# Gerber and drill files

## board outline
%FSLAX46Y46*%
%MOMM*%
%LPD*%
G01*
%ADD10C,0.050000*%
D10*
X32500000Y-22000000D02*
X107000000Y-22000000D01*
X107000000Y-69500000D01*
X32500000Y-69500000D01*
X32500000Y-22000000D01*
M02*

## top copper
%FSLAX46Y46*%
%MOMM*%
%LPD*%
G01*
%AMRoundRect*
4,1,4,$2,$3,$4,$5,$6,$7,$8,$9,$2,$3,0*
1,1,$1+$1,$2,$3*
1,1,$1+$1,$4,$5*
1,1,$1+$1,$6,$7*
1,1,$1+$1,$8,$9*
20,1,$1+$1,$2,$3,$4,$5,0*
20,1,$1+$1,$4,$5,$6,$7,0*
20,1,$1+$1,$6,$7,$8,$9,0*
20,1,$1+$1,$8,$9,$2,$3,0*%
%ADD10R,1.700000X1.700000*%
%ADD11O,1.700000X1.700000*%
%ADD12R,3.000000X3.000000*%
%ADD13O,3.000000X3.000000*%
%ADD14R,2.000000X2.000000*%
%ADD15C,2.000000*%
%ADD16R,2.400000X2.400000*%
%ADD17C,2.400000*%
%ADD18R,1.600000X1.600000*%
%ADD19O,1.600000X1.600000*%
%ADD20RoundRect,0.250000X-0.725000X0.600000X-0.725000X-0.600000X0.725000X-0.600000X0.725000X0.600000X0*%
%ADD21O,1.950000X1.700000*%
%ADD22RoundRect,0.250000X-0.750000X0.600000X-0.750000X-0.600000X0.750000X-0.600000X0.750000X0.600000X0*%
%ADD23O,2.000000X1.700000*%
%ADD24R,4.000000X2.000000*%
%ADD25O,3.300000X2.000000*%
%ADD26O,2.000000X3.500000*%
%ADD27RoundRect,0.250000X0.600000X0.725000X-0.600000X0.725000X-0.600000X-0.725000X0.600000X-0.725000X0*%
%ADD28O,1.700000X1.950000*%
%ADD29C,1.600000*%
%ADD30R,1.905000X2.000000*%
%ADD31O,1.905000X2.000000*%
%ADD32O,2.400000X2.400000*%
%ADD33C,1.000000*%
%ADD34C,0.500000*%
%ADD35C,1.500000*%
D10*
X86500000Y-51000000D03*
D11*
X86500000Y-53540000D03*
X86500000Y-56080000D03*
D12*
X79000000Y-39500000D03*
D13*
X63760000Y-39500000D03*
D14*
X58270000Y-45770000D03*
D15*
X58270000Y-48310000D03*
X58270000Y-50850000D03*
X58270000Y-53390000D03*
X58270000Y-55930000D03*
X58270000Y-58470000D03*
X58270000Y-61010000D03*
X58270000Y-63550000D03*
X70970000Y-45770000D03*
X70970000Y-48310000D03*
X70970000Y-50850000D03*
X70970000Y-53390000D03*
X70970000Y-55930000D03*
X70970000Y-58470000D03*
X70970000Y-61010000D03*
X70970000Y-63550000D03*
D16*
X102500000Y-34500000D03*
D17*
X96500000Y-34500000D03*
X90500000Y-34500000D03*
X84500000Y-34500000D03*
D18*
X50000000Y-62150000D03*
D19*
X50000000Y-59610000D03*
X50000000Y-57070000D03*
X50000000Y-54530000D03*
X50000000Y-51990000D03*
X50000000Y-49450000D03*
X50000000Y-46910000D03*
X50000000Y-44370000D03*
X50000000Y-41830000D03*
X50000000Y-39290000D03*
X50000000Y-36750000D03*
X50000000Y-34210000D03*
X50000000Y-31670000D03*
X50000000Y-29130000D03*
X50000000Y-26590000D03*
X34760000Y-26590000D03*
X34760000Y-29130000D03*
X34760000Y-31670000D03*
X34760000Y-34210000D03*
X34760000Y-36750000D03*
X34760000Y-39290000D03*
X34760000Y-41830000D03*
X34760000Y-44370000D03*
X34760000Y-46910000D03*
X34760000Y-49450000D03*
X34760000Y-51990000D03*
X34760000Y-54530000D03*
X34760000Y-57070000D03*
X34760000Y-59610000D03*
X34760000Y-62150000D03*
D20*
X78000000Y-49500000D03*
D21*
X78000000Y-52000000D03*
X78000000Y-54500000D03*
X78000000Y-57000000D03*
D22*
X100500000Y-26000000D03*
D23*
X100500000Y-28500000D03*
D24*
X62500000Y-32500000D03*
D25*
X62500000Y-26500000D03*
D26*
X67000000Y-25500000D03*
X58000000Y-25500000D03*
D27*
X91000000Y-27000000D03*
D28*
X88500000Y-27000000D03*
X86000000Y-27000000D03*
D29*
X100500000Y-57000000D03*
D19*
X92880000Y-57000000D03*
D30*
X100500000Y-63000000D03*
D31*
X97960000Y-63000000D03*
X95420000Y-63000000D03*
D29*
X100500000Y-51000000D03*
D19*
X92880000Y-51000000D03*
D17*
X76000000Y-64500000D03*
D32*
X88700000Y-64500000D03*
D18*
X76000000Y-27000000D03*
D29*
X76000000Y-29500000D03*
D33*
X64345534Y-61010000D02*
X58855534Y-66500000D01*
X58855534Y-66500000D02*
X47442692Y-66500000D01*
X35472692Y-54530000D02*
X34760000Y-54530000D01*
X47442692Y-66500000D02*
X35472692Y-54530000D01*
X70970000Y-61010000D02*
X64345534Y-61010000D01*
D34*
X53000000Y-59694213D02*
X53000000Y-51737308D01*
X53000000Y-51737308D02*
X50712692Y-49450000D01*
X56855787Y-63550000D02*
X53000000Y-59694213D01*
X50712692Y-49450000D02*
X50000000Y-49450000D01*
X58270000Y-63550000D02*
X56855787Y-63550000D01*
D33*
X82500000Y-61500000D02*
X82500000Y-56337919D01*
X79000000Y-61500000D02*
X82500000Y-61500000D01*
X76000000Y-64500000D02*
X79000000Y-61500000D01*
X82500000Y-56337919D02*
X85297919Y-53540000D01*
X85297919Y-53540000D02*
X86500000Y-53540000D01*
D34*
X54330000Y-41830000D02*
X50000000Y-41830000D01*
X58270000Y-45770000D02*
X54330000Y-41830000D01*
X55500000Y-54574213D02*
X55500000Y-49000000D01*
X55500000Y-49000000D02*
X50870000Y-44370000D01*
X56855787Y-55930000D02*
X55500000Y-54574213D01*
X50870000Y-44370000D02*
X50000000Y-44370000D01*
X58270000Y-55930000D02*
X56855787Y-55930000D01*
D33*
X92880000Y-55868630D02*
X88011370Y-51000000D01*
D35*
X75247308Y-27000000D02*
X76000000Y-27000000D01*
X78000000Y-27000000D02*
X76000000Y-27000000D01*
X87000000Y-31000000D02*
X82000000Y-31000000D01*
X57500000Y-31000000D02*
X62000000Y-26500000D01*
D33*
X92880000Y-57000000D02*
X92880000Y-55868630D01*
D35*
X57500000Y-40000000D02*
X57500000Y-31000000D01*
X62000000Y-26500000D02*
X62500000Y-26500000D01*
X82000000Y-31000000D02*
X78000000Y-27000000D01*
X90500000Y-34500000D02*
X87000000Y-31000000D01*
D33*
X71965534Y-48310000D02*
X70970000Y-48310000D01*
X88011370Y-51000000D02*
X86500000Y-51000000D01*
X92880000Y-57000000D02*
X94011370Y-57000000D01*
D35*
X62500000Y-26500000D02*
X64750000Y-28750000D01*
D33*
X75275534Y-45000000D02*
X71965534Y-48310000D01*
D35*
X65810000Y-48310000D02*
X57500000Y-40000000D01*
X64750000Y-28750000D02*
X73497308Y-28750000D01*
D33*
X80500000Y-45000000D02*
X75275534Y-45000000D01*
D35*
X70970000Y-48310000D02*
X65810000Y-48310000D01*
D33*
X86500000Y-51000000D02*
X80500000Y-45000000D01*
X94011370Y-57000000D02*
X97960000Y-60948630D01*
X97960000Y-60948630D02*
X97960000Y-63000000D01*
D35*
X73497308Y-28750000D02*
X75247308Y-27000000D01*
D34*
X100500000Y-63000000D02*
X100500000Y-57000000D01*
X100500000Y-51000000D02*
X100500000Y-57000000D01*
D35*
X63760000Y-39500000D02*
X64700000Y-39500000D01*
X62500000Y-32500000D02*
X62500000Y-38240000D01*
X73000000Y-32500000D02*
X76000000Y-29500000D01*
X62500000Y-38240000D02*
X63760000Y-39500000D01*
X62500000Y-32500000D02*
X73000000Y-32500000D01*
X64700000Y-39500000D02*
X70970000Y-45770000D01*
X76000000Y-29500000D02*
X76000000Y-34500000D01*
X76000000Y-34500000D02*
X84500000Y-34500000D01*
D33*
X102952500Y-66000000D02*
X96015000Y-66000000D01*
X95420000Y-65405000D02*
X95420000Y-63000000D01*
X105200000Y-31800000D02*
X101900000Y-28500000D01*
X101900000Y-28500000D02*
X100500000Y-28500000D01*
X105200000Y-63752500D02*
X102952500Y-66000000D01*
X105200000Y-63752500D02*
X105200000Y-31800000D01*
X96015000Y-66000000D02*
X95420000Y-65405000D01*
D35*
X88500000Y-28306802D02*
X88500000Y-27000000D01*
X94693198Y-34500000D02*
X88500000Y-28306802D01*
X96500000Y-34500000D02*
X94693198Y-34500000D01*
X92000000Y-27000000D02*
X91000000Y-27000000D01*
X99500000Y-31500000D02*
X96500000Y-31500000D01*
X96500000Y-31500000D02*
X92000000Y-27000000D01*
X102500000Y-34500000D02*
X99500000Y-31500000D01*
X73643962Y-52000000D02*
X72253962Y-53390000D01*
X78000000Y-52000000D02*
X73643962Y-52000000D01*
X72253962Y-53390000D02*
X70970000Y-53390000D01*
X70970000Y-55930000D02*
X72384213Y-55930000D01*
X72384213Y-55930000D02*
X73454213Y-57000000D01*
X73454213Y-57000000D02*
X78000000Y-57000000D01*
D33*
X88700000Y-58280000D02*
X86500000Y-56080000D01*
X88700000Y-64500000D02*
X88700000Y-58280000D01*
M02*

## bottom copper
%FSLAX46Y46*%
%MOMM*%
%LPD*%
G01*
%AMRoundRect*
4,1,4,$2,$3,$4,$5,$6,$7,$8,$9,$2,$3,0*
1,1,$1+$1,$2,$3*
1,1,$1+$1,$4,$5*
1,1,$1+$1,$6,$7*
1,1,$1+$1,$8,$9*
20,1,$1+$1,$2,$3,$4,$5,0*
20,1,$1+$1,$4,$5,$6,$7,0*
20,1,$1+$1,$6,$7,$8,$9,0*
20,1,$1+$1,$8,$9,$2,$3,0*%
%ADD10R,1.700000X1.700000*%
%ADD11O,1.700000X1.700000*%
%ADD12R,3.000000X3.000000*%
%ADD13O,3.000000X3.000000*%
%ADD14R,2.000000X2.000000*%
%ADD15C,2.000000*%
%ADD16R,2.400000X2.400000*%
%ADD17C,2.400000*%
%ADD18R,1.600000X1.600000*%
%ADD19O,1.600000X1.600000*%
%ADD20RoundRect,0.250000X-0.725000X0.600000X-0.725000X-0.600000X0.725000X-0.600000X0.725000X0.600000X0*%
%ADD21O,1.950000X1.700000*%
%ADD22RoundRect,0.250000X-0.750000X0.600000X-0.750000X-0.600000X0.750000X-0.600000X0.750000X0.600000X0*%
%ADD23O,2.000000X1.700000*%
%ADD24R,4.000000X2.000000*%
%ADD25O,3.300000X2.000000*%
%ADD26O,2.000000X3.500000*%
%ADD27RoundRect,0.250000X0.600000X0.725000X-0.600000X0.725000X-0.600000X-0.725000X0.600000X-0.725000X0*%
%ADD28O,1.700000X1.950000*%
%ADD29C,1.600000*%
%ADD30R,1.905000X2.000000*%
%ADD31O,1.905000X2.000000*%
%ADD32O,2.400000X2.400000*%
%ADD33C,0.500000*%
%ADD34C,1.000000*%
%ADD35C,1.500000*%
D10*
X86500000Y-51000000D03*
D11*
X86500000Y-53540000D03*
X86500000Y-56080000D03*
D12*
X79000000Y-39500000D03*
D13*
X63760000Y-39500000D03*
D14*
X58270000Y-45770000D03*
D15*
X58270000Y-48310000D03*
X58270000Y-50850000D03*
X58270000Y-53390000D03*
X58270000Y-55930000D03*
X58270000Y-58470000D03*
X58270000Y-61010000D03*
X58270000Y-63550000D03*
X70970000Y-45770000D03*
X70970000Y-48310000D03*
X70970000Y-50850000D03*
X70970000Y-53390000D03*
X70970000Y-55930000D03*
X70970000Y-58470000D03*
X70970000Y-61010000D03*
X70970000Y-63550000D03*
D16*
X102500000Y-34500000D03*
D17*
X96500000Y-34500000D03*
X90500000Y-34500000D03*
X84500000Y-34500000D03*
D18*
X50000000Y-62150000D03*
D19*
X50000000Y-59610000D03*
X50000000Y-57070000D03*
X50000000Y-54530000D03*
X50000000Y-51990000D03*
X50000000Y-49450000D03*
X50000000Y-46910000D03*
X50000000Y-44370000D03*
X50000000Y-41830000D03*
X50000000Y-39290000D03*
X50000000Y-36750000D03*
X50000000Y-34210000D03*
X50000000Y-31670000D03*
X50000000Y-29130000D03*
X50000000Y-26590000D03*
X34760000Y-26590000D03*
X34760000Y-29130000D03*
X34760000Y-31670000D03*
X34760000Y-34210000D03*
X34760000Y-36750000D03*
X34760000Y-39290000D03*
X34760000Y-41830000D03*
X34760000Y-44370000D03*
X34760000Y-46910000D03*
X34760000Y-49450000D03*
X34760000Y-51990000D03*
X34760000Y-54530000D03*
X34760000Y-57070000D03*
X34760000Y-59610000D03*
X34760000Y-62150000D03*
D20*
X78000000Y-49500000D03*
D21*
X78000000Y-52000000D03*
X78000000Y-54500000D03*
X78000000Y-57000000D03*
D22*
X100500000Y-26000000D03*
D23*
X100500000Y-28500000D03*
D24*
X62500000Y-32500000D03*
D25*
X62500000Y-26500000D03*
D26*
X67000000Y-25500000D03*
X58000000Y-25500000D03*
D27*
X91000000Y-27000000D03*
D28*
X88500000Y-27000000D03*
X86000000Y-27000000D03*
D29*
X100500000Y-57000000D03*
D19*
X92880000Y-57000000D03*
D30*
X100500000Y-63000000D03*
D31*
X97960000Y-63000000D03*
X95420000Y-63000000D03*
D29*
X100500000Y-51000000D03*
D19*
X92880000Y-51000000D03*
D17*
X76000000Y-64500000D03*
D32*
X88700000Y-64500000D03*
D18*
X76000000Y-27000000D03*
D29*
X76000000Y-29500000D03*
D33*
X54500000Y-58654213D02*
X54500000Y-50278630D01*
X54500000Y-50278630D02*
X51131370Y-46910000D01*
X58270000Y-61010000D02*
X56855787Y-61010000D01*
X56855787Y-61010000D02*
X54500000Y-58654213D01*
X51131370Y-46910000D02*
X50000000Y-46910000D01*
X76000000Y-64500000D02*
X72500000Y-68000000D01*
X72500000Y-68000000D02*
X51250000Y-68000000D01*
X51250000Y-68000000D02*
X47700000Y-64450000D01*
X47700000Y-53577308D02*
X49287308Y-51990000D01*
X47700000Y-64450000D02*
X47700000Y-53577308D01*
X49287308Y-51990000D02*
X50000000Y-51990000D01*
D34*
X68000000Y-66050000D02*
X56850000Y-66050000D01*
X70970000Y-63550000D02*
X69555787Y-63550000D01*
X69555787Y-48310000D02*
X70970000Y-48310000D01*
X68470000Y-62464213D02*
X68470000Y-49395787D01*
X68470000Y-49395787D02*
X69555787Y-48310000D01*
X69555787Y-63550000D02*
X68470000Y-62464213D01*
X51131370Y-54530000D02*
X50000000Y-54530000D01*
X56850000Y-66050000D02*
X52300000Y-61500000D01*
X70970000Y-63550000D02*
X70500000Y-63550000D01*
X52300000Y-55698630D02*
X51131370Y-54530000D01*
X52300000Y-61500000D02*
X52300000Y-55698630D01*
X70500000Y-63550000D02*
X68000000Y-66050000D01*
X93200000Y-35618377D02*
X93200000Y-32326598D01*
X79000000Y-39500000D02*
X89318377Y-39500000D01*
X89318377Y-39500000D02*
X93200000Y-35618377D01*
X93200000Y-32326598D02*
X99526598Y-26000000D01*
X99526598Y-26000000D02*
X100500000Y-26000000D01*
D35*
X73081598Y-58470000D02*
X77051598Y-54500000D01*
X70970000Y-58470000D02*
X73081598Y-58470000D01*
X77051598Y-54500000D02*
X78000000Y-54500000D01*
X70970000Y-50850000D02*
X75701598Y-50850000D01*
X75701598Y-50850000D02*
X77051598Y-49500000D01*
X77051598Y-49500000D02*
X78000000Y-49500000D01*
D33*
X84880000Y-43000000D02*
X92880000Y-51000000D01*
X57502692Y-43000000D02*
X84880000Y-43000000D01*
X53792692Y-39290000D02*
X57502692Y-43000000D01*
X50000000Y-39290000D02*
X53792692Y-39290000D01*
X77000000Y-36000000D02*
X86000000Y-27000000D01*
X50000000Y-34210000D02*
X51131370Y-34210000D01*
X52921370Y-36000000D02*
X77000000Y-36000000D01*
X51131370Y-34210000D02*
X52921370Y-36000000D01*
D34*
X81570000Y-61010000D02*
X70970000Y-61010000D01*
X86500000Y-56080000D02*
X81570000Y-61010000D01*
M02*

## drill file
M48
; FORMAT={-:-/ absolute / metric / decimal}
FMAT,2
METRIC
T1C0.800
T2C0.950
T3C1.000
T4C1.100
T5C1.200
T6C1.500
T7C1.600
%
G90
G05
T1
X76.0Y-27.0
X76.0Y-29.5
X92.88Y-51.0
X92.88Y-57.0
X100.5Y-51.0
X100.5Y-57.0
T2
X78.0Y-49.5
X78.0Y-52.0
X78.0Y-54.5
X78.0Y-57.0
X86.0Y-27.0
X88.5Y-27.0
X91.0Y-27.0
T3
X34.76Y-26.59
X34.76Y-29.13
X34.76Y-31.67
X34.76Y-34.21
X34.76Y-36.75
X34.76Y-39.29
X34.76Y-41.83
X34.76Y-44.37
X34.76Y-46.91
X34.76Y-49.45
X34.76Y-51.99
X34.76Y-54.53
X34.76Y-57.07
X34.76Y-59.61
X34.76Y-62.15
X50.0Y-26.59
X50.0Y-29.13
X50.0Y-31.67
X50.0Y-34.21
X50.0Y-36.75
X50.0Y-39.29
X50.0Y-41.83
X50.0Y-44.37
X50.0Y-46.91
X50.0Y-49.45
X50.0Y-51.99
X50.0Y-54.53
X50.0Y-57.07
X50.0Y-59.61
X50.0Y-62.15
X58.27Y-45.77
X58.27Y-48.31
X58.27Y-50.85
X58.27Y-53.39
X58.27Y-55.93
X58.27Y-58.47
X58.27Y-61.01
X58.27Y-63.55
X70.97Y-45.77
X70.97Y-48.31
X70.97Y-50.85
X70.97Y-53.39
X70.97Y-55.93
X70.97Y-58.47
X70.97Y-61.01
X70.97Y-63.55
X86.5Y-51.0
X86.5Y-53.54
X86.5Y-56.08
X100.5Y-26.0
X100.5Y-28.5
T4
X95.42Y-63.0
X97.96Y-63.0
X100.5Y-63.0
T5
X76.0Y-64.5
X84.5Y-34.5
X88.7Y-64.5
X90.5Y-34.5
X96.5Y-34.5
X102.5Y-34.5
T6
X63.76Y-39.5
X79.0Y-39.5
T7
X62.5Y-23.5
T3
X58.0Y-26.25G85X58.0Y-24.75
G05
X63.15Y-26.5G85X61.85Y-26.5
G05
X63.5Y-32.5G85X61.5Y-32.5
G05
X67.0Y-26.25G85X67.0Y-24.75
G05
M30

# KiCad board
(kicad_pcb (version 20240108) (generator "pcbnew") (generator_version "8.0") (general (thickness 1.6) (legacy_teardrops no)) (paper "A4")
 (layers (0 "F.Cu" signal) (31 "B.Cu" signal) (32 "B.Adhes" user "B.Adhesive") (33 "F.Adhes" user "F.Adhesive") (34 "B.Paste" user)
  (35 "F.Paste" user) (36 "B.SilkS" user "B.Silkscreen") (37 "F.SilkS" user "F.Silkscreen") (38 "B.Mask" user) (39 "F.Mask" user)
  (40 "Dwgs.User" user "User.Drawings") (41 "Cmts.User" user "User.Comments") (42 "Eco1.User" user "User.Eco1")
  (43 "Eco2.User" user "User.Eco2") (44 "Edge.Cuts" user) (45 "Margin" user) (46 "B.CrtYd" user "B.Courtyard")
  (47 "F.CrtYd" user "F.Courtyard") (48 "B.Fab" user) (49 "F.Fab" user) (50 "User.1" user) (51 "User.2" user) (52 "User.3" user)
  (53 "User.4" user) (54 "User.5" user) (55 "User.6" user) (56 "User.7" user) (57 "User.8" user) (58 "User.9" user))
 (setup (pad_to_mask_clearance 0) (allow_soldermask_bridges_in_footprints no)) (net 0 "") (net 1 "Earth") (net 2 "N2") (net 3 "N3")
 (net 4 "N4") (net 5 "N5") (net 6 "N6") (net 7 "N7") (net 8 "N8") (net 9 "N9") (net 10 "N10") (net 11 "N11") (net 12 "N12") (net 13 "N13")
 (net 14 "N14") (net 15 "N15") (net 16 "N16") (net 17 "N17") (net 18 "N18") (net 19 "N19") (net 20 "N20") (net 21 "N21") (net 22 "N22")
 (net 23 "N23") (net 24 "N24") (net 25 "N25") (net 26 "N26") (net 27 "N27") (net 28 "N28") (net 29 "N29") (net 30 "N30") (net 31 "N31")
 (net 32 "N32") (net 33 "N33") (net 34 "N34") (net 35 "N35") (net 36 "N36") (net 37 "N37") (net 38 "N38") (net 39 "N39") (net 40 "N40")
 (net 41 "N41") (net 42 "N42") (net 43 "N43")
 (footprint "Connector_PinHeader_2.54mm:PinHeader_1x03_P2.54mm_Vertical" (layer "F.Cu") (at 86.5 51)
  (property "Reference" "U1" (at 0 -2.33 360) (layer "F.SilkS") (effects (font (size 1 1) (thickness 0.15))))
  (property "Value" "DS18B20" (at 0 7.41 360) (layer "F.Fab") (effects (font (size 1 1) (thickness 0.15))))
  (pad "1" thru_hole rect (at 0 0) (size 1.7 1.7) (drill 1) (layers "*.Cu" "*.Mask") (remove_unused_layers no) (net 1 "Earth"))
  (pad "2" thru_hole oval (at 0 2.54) (size 1.7 1.7) (drill 1) (layers "*.Cu" "*.Mask") (remove_unused_layers no) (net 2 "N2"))
  (pad "3" thru_hole oval (at 0 5.08) (size 1.7 1.7) (drill 1) (layers "*.Cu" "*.Mask") (remove_unused_layers no) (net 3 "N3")))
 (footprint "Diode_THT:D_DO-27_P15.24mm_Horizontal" (layer "F.Cu") (at 79 39.5 180)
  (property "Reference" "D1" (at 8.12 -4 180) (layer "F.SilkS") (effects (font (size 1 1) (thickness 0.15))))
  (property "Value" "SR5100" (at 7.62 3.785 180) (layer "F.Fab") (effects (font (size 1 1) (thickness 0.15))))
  (pad "1" thru_hole rect (at 0 0 180) (size 3 3) (drill 1.5) (layers "*.Cu" "*.Mask") (remove_unused_layers no) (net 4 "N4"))
  (pad "2" thru_hole oval (at 15.24 0 180) (size 3 3) (drill 1.5) (layers "*.Cu" "*.Mask") (remove_unused_layers no) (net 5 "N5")))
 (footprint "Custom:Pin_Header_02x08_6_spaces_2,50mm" (layer "F.Cu") (at 57 44.5)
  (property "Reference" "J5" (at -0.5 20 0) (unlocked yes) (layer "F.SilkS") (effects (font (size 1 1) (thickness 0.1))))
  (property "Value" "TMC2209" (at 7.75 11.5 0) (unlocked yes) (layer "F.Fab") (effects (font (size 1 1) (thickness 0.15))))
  (pad "1" thru_hole rect (at 1.27 1.27) (size 2 2) (drill 1) (layers "*.Cu" "*.Mask") (remove_unused_layers no) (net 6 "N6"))
  (pad "2" thru_hole circle (at 1.27 3.81) (size 2 2) (drill 1) (layers "*.Cu" "*.Mask") (remove_unused_layers no) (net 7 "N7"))
  (pad "3" thru_hole circle (at 1.27 6.35) (size 2 2) (drill 1) (layers "*.Cu" "*.Mask") (remove_unused_layers no) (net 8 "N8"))
  (pad "4" thru_hole circle (at 1.27 8.89) (size 2 2) (drill 1) (layers "*.Cu" "*.Mask") (remove_unused_layers no) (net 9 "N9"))
  (pad "5" thru_hole circle (at 1.27 11.43) (size 2 2) (drill 1) (layers "*.Cu" "*.Mask") (remove_unused_layers no) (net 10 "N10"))
  (pad "6" thru_hole circle (at 1.27 13.97) (size 2 2) (drill 1) (layers "*.Cu" "*.Mask") (remove_unused_layers no) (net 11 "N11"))
  (pad "7" thru_hole circle (at 1.27 16.51) (size 2 2) (drill 1) (layers "*.Cu" "*.Mask") (remove_unused_layers no) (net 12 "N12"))
  (pad "8" thru_hole circle (at 1.27 19.05) (size 2 2) (drill 1) (layers "*.Cu" "*.Mask") (remove_unused_layers no) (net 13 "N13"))
  (pad "9" thru_hole circle (at 13.97 1.27) (size 2 2) (drill 1) (layers "*.Cu" "*.Mask") (remove_unused_layers no) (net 5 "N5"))
  (pad "10" thru_hole circle (at 13.97 3.81) (size 2 2) (drill 1) (layers "*.Cu" "*.Mask") (remove_unused_layers no) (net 1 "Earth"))
  (pad "11" thru_hole circle (at 13.97 6.35) (size 2 2) (drill 1) (layers "*.Cu" "*.Mask") (remove_unused_layers no) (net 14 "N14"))
  (pad "12" thru_hole circle (at 13.97 8.89) (size 2 2) (drill 1) (layers "*.Cu" "*.Mask") (remove_unused_layers no) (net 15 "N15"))
  (pad "13" thru_hole circle (at 13.97 11.43) (size 2 2) (drill 1) (layers "*.Cu" "*.Mask") (remove_unused_layers no) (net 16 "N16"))
  (pad "14" thru_hole circle (at 13.97 13.97) (size 2 2) (drill 1) (layers "*.Cu" "*.Mask") (remove_unused_layers no) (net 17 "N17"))
  (pad "15" thru_hole circle (at 13.97 16.51) (size 2 2) (drill 1) (layers "*.Cu" "*.Mask") (remove_unused_layers no) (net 3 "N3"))
  (pad "16" thru_hole circle (at 13.97 19.05) (size 2 2) (drill 1) (layers "*.Cu" "*.Mask") (remove_unused_layers no) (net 1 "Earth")))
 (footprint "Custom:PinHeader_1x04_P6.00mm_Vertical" (layer "F.Cu") (at 102.5 34.5 -90)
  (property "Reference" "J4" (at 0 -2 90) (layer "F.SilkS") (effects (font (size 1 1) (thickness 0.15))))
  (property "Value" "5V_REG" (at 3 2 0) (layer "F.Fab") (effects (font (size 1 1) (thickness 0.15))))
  (pad "1" thru_hole rect (at 0 0 270) (size 2.4 2.4) (drill 1.2) (layers "*.Cu" "*.Mask") (remove_unused_layers no) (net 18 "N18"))
  (pad "2" thru_hole circle (at 0 6 270) (size 2.4 2.4) (drill 1.2) (layers "*.Cu" "*.Mask") (remove_unused_layers no) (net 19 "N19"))
  (pad "3" thru_hole circle (at 0 12 270) (size 2.4 2.4) (drill 1.2) (layers "*.Cu" "*.Mask") (remove_unused_layers no) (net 1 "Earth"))
  (pad "4" thru_hole circle (at 0 18 270) (size 2.4 2.4) (drill 1.2) (layers "*.Cu" "*.Mask") (remove_unused_layers no) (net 5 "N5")))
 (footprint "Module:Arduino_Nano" (layer "F.Cu") (at 50 62.15 180)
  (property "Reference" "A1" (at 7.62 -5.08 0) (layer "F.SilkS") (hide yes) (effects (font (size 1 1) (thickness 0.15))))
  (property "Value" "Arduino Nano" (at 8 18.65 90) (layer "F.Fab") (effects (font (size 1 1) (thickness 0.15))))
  (pad "1" thru_hole rect (at 0 0 180) (size 1.6 1.6) (drill 1) (layers "*.Cu" "*.Mask") (remove_unused_layers no) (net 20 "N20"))
  (pad "2" thru_hole oval (at 0 2.54 180) (size 1.6 1.6) (drill 1) (layers "*.Cu" "*.Mask") (remove_unused_layers no) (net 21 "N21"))
  (pad "3" thru_hole oval (at 0 5.08 180) (size 1.6 1.6) (drill 1) (layers "*.Cu" "*.Mask") (remove_unused_layers no) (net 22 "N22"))
  (pad "4" thru_hole oval (at 0 7.62 180) (size 1.6 1.6) (drill 1) (layers "*.Cu" "*.Mask") (remove_unused_layers no) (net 1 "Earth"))
  (pad "5" thru_hole oval (at 0 10.16 180) (size 1.6 1.6) (drill 1) (layers "*.Cu" "*.Mask") (remove_unused_layers no) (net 2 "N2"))
  (pad "6" thru_hole oval (at 0 12.7 180) (size 1.6 1.6) (drill 1) (layers "*.Cu" "*.Mask") (remove_unused_layers no) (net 13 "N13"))
  (pad "7" thru_hole oval (at 0 15.24 180) (size 1.6 1.6) (drill 1) (layers "*.Cu" "*.Mask") (remove_unused_layers no) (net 12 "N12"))
  (pad "8" thru_hole oval (at 0 17.78 180) (size 1.6 1.6) (drill 1) (layers "*.Cu" "*.Mask") (remove_unused_layers no) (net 10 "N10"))
  (pad "9" thru_hole oval (at 0 20.32 180) (size 1.6 1.6) (drill 1) (layers "*.Cu" "*.Mask") (remove_unused_layers no) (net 6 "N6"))
  (pad "10" thru_hole oval (at 0 22.86 180) (size 1.6 1.6) (drill 1) (layers "*.Cu" "*.Mask") (remove_unused_layers no) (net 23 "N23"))
  (pad "11" thru_hole oval (at 0 25.4 180) (size 1.6 1.6) (drill 1) (layers "*.Cu" "*.Mask") (remove_unused_layers no) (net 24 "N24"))
  (pad "12" thru_hole oval (at 0 27.94 180) (size 1.6 1.6) (drill 1) (layers "*.Cu" "*.Mask") (remove_unused_layers no) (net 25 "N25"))
  (pad "13" thru_hole oval (at 0 30.48 180) (size 1.6 1.6) (drill 1) (layers "*.Cu" "*.Mask") (remove_unused_layers no) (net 25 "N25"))
  (pad "14" thru_hole oval (at 0 33.02 180) (size 1.6 1.6) (drill 1) (layers "*.Cu" "*.Mask") (remove_unused_layers no) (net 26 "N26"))
  (pad "15" thru_hole oval (at 0 35.56 180) (size 1.6 1.6) (drill 1) (layers "*.Cu" "*.Mask") (remove_unused_layers no) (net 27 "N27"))
  (pad "16" thru_hole oval (at 15.24 35.56 180) (size 1.6 1.6) (drill 1) (layers "*.Cu" "*.Mask") (remove_unused_layers no) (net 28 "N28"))
  (pad "17" thru_hole oval (at 15.24 33.02 180) (size 1.6 1.6) (drill 1) (layers "*.Cu" "*.Mask") (remove_unused_layers no) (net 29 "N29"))
  (pad "18" thru_hole oval (at 15.24 30.48 180) (size 1.6 1.6) (drill 1) (layers "*.Cu" "*.Mask") (remove_unused_layers no) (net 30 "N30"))
  (pad "19" thru_hole oval (at 15.24 27.94 180) (size 1.6 1.6) (drill 1) (layers "*.Cu" "*.Mask") (remove_unused_layers no) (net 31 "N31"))
  (pad "20" thru_hole oval (at 15.24 25.4 180) (size 1.6 1.6) (drill 1) (layers "*.Cu" "*.Mask") (remove_unused_layers no) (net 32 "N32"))
  (pad "21" thru_hole oval (at 15.24 22.86 180) (size 1.6 1.6) (drill 1) (layers "*.Cu" "*.Mask") (remove_unused_layers no) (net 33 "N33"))
  (pad "22" thru_hole oval (at 15.24 20.32 180) (size 1.6 1.6) (drill 1) (layers "*.Cu" "*.Mask") (remove_unused_layers no) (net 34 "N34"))
  (pad "23" thru_hole oval (at 15.24 17.78 180) (size 1.6 1.6) (drill 1) (layers "*.Cu" "*.Mask") (remove_unused_layers no) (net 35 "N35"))
  (pad "24" thru_hole oval (at 15.24 15.24 180) (size 1.6 1.6) (drill 1) (layers "*.Cu" "*.Mask") (remove_unused_layers no) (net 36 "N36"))
  (pad "25" thru_hole oval (at 15.24 12.7 180) (size 1.6 1.6) (drill 1) (layers "*.Cu" "*.Mask") (remove_unused_layers no) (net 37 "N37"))
  (pad "26" thru_hole oval (at 15.24 10.16 180) (size 1.6 1.6) (drill 1) (layers "*.Cu" "*.Mask") (remove_unused_layers no) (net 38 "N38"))
  (pad "27" thru_hole oval (at 15.24 7.62 180) (size 1.6 1.6) (drill 1) (layers "*.Cu" "*.Mask") (remove_unused_layers no) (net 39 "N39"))
  (pad "28" thru_hole oval (at 15.24 5.08 180) (size 1.6 1.6) (drill 1) (layers "*.Cu" "*.Mask") (remove_unused_layers no) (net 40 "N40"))
  (pad "29" thru_hole oval (at 15.24 2.54 180) (size 1.6 1.6) (drill 1) (layers "*.Cu" "*.Mask") (remove_unused_layers no) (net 1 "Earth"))
  (pad "30" thru_hole oval (at 15.24 0 180) (size 1.6 1.6) (drill 1) (layers "*.Cu" "*.Mask") (remove_unused_layers no) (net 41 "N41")))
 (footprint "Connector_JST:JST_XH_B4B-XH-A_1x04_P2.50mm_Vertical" (layer "F.Cu") (at 78 49.5 -90)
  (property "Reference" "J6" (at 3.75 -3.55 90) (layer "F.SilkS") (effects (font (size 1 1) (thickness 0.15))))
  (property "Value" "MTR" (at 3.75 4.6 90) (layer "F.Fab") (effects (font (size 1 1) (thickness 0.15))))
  (pad "1" thru_hole roundrect (at 0 0 270) (size 1.7 1.95) (drill 0.95) (layers "*.Cu" "*.Mask") (remove_unused_layers no)
   (roundrect_rratio 0.147059) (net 14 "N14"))
  (pad "2" thru_hole oval (at 2.5 0 270) (size 1.7 1.95) (drill 0.95) (layers "*.Cu" "*.Mask") (remove_unused_layers no) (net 15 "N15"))
  (pad "3" thru_hole oval (at 5 0 270) (size 1.7 1.95) (drill 0.95) (layers "*.Cu" "*.Mask") (remove_unused_layers no) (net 17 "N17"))
  (pad "4" thru_hole oval (at 7.5 0 270) (size 1.7 1.95) (drill 0.95) (layers "*.Cu" "*.Mask") (remove_unused_layers no) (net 16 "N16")))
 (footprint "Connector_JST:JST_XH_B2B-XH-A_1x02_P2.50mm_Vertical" (layer "F.Cu") (at 100.5 26 -90)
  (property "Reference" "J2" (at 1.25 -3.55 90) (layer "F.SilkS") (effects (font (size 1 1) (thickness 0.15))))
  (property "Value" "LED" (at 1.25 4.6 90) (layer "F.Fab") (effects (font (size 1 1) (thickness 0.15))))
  (pad "1" thru_hole roundrect (at 0 0 270) (size 1.7 2) (drill 1) (layers "*.Cu" "*.Mask") (remove_unused_layers no)
   (roundrect_rratio 0.147059) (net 4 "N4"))
  (pad "2" thru_hole oval (at 2.5 0 270) (size 1.7 2) (drill 1) (layers "*.Cu" "*.Mask") (remove_unused_layers no) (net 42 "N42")))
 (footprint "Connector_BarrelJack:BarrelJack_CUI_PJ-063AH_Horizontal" (layer "F.Cu") (at 62.5 32.5 180)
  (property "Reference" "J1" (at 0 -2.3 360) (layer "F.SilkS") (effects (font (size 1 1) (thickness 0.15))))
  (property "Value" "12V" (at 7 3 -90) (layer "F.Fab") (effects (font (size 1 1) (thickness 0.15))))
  (pad "" np_thru_hole circle (at 0 9 180) (size 1.6 1.6) (drill 1.6) (layers "F&B.Cu" "*.Mask"))
  (pad "1" thru_hole rect (at 0 0 180) (size 4 2) (drill oval 3 1) (layers "*.Cu" "*.Mask") (remove_unused_layers no) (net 5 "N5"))
  (pad "2" thru_hole oval (at 0 6 180) (size 3.3 2) (drill oval 2.3 1) (layers "*.Cu" "*.Mask") (remove_unused_layers no) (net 1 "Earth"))
  (pad "MP" thru_hole oval (at -4.5 7 180) (size 2 3.5) (drill oval 1 2.5) (layers "*.Cu" "*.Mask") (remove_unused_layers no))
  (pad "MP" thru_hole oval (at 4.5 7 180) (size 2 3.5) (drill oval 1 2.5) (layers "*.Cu" "*.Mask") (remove_unused_layers no)))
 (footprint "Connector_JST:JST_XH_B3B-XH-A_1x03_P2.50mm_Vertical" (layer "F.Cu") (at 91 27 180)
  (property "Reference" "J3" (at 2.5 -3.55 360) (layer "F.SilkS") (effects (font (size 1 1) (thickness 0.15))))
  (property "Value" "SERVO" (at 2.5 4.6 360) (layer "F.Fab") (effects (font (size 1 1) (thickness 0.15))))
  (pad "1" thru_hole roundrect (at 0 0 180) (size 1.7 1.95) (drill 0.95) (layers "*.Cu" "*.Mask") (remove_unused_layers no)
   (roundrect_rratio 0.147059) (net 18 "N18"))
  (pad "2" thru_hole oval (at 2.5 0 180) (size 1.7 1.95) (drill 0.95) (layers "*.Cu" "*.Mask") (remove_unused_layers no) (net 19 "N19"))
  (pad "3" thru_hole oval (at 5 0 180) (size 1.7 1.95) (drill 0.95) (layers "*.Cu" "*.Mask") (remove_unused_layers no) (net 25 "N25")))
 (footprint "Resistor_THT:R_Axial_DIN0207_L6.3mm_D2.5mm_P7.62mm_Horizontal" (layer "F.Cu") (at 100.5 57 180)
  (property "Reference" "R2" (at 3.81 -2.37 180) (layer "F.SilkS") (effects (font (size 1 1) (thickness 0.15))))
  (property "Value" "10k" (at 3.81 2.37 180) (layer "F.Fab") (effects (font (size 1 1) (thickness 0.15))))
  (pad "1" thru_hole circle (at 0 0 180) (size 1.6 1.6) (drill 0.8) (layers "*.Cu" "*.Mask") (remove_unused_layers no) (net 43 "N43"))
  (pad "2" thru_hole oval (at 7.62 0 180) (size 1.6 1.6) (drill 0.8) (layers "*.Cu" "*.Mask") (remove_unused_layers no) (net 1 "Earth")))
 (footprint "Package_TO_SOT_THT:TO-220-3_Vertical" (layer "F.Cu") (at 100.5 63 180)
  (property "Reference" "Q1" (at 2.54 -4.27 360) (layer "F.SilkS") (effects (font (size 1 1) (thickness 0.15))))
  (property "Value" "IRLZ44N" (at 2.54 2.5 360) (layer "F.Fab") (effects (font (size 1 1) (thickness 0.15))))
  (pad "1" thru_hole rect (at 0 0 180) (size 1.905 2) (drill 1.1) (layers "*.Cu" "*.Mask") (remove_unused_layers no) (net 43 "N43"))
  (pad "2" thru_hole oval (at 2.54 0 180) (size 1.905 2) (drill 1.1) (layers "*.Cu" "*.Mask") (remove_unused_layers no) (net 1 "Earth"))
  (pad "3" thru_hole oval (at 5.08 0 180) (size 1.905 2) (drill 1.1) (layers "*.Cu" "*.Mask") (remove_unused_layers no) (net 42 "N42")))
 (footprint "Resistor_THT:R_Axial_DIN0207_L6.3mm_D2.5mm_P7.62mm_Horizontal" (layer "F.Cu") (at 100.5 51 180)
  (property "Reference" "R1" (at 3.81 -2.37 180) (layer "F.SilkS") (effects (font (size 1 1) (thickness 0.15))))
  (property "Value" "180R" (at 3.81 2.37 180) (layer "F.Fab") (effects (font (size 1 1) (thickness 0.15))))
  (pad "1" thru_hole circle (at 0 0 180) (size 1.6 1.6) (drill 0.8) (layers "*.Cu" "*.Mask") (remove_unused_layers no) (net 43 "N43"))
  (pad "2" thru_hole oval (at 7.62 0 180) (size 1.6 1.6) (drill 0.8) (layers "*.Cu" "*.Mask") (remove_unused_layers no) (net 23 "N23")))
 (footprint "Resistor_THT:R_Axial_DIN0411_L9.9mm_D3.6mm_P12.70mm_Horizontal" (layer "F.Cu") (at 76 64.5)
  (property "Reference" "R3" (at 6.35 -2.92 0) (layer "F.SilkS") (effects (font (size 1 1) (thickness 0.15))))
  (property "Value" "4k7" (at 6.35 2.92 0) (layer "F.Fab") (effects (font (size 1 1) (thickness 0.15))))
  (pad "1" thru_hole circle (at 0 0) (size 2.4 2.4) (drill 1.2) (layers "*.Cu" "*.Mask") (remove_unused_layers no) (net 2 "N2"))
  (pad "2" thru_hole oval (at 12.7 0) (size 2.4 2.4) (drill 1.2) (layers "*.Cu" "*.Mask") (remove_unused_layers no) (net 3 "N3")))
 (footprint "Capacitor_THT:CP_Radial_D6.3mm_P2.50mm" (layer "F.Cu") (at 76 27 -90)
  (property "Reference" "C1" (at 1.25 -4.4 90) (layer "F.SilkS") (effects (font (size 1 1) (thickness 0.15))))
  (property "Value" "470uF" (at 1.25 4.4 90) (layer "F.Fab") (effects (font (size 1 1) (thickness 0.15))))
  (pad "1" thru_hole rect (at 0 0 270) (size 1.6 1.6) (drill 0.8) (layers "*.Cu" "*.Mask") (remove_unused_layers no) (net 1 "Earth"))
  (pad "2" thru_hole circle (at 2.5 0 270) (size 1.6 1.6) (drill 0.8) (layers "*.Cu" "*.Mask") (remove_unused_layers no) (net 5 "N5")))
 (gr_rect (start 32.5 22) (end 107 69.5) (stroke (width 0.05) (type default)) (fill none) (layer "Edge.Cuts"))
 (segment (start 64.345534 61.01) (end 58.855534 66.5) (width 1) (layer "F.Cu") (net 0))
 (segment (start 58.855534 66.5) (end 47.442692 66.5) (width 1) (layer "F.Cu") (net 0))
 (segment (start 35.472692 54.53) (end 34.76 54.53) (width 1) (layer "F.Cu") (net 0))
 (segment (start 47.442692 66.5) (end 35.472692 54.53) (width 1) (layer "F.Cu") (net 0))
 (segment (start 70.97 61.01) (end 64.345534 61.01) (width 1) (layer "F.Cu") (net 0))
 (segment (start 54.5 58.654213) (end 54.5 50.27863) (width 0.5) (layer "B.Cu") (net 12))
 (segment (start 54.5 50.27863) (end 51.13137 46.91) (width 0.5) (layer "B.Cu") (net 12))
 (segment (start 58.27 61.01) (end 56.855787 61.01) (width 0.5) (layer "B.Cu") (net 12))
 (segment (start 56.855787 61.01) (end 54.5 58.654213) (width 0.5) (layer "B.Cu") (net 12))
 (segment (start 51.13137 46.91) (end 50 46.91) (width 0.5) (layer "B.Cu") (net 12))
 (segment (start 53 59.694213) (end 53 51.737308) (width 0.5) (layer "F.Cu") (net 13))
 (segment (start 53 51.737308) (end 50.712692 49.45) (width 0.5) (layer "F.Cu") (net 13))
 (segment (start 56.855787 63.55) (end 53 59.694213) (width 0.5) (layer "F.Cu") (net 13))
 (segment (start 50.712692 49.45) (end 50 49.45) (width 0.5) (layer "F.Cu") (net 13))
 (segment (start 58.27 63.55) (end 56.855787 63.55) (width 0.5) (layer "F.Cu") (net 13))
 (segment (start 82.5 61.5) (end 82.5 56.337919) (width 1) (layer "F.Cu") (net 2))
 (segment (start 79 61.5) (end 82.5 61.5) (width 1) (layer "F.Cu") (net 2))
 (segment (start 76 64.5) (end 79 61.5) (width 1) (layer "F.Cu") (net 2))
 (segment (start 82.5 56.337919) (end 85.297919 53.54) (width 1) (layer "F.Cu") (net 2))
 (segment (start 85.297919 53.54) (end 86.5 53.54) (width 1) (layer "F.Cu") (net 2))
 (segment (start 76 64.5) (end 72.5 68) (width 0.5) (layer "B.Cu") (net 2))
 (segment (start 72.5 68) (end 51.25 68) (width 0.5) (layer "B.Cu") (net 2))
 (segment (start 51.25 68) (end 47.7 64.45) (width 0.5) (layer "B.Cu") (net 2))
 (segment (start 47.7 53.577308) (end 49.287308 51.99) (width 0.5) (layer "B.Cu") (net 2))
 (segment (start 47.7 64.45) (end 47.7 53.577308) (width 0.5) (layer "B.Cu") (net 2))
 (segment (start 49.287308 51.99) (end 50 51.99) (width 0.5) (layer "B.Cu") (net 2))
 (segment (start 54.33 41.83) (end 50 41.83) (width 0.5) (layer "F.Cu") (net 6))
 (segment (start 58.27 45.77) (end 54.33 41.83) (width 0.5) (layer "F.Cu") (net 6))
 (segment (start 55.5 54.574213) (end 55.5 49) (width 0.5) (layer "F.Cu") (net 10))
 (segment (start 55.5 49) (end 50.87 44.37) (width 0.5) (layer "F.Cu") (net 10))
 (segment (start 56.855787 55.93) (end 55.5 54.574213) (width 0.5) (layer "F.Cu") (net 10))
 (segment (start 50.87 44.37) (end 50 44.37) (width 0.5) (layer "F.Cu") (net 10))
 (segment (start 58.27 55.93) (end 56.855787 55.93) (width 0.5) (layer "F.Cu") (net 10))
 (segment (start 92.88 55.86863) (end 88.01137 51) (width 1) (layer "F.Cu") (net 1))
 (segment (start 75.247308 27) (end 76 27) (width 1.5) (layer "F.Cu") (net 1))
 (segment (start 78 27) (end 76 27) (width 1.5) (layer "F.Cu") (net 1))
 (segment (start 87 31) (end 82 31) (width 1.5) (layer "F.Cu") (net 1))
 (segment (start 57.5 31) (end 62 26.5) (width 1.5) (layer "F.Cu") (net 1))
 (segment (start 92.88 57) (end 92.88 55.86863) (width 1) (layer "F.Cu") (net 1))
 (segment (start 57.5 40) (end 57.5 31) (width 1.5) (layer "F.Cu") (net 1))
 (segment (start 62 26.5) (end 62.5 26.5) (width 1.5) (layer "F.Cu") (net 1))
 (segment (start 82 31) (end 78 27) (width 1.5) (layer "F.Cu") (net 1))
 (segment (start 90.5 34.5) (end 87 31) (width 1.5) (layer "F.Cu") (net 1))
 (segment (start 71.965534 48.31) (end 70.97 48.31) (width 1) (layer "F.Cu") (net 1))
 (segment (start 88.01137 51) (end 86.5 51) (width 1) (layer "F.Cu") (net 1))
 (segment (start 92.88 57) (end 94.01137 57) (width 1) (layer "F.Cu") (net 1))
 (segment (start 62.5 26.5) (end 64.75 28.75) (width 1.5) (layer "F.Cu") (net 1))
 (segment (start 75.275534 45) (end 71.965534 48.31) (width 1) (layer "F.Cu") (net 1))
 (segment (start 65.81 48.31) (end 57.5 40) (width 1.5) (layer "F.Cu") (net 1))
 (segment (start 64.75 28.75) (end 73.497308 28.75) (width 1.5) (layer "F.Cu") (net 1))
 (segment (start 80.5 45) (end 75.275534 45) (width 1) (layer "F.Cu") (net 1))
 (segment (start 70.97 48.31) (end 65.81 48.31) (width 1.5) (layer "F.Cu") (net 1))
 (segment (start 86.5 51) (end 80.5 45) (width 1) (layer "F.Cu") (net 1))
 (segment (start 94.01137 57) (end 97.96 60.94863) (width 1) (layer "F.Cu") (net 1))
 (segment (start 97.96 60.94863) (end 97.96 63) (width 1) (layer "F.Cu") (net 1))
 (segment (start 73.497308 28.75) (end 75.247308 27) (width 1.5) (layer "F.Cu") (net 1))
 (segment (start 68 66.05) (end 56.85 66.05) (width 1) (layer "B.Cu") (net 1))
 (segment (start 70.97 63.55) (end 69.555787 63.55) (width 1) (layer "B.Cu") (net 1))
 (segment (start 69.555787 48.31) (end 70.97 48.31) (width 1) (layer "B.Cu") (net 1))
 (segment (start 68.47 62.464213) (end 68.47 49.395787) (width 1) (layer "B.Cu") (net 1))
 (segment (start 68.47 49.395787) (end 69.555787 48.31) (width 1) (layer "B.Cu") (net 1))
 (segment (start 69.555787 63.55) (end 68.47 62.464213) (width 1) (layer "B.Cu") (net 1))
 (segment (start 51.13137 54.53) (end 50 54.53) (width 1) (layer "B.Cu") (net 1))
 (segment (start 56.85 66.05) (end 52.3 61.5) (width 1) (layer "B.Cu") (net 1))
 (segment (start 70.97 63.55) (end 70.5 63.55) (width 1) (layer "B.Cu") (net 1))
 (segment (start 52.3 55.69863) (end 51.13137 54.53) (width 1) (layer "B.Cu") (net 1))
 (segment (start 52.3 61.5) (end 52.3 55.69863) (width 1) (layer "B.Cu") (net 1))
 (segment (start 70.5 63.55) (end 68 66.05) (width 1) (layer "B.Cu") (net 1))
 (segment (start 93.2 35.618377) (end 93.2 32.326598) (width 1) (layer "B.Cu") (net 4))
 (segment (start 79 39.5) (end 89.318377 39.5) (width 1) (layer "B.Cu") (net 4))
 (segment (start 89.318377 39.5) (end 93.2 35.618377) (width 1) (layer "B.Cu") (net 4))
 (segment (start 93.2 32.326598) (end 99.526598 26) (width 1) (layer "B.Cu") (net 4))
 (segment (start 99.526598 26) (end 100.5 26) (width 1) (layer "B.Cu") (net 4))
 (segment (start 100.5 63) (end 100.5 57) (width 0.5) (layer "F.Cu") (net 43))
 (segment (start 100.5 51) (end 100.5 57) (width 0.5) (layer "F.Cu") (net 43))
 (segment (start 63.76 39.5) (end 64.7 39.5) (width 1.5) (layer "F.Cu") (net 5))
 (segment (start 62.5 32.5) (end 62.5 38.24) (width 1.5) (layer "F.Cu") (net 5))
 (segment (start 73 32.5) (end 76 29.5) (width 1.5) (layer "F.Cu") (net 5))
 (segment (start 62.5 38.24) (end 63.76 39.5) (width 1.5) (layer "F.Cu") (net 5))
 (segment (start 62.5 32.5) (end 73 32.5) (width 1.5) (layer "F.Cu") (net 5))
 (segment (start 64.7 39.5) (end 70.97 45.77) (width 1.5) (layer "F.Cu") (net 5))
 (segment (start 76 29.5) (end 76 34.5) (width 1.5) (layer "F.Cu") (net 5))
 (segment (start 76 34.5) (end 84.5 34.5) (width 1.5) (layer "F.Cu") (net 5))
 (segment (start 102.9525 66) (end 96.015 66) (width 1) (layer "F.Cu") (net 42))
 (segment (start 95.42 65.405) (end 95.42 63) (width 1) (layer "F.Cu") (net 42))
 (segment (start 105.2 31.8) (end 101.9 28.5) (width 1) (layer "F.Cu") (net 42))
 (segment (start 101.9 28.5) (end 100.5 28.5) (width 1) (layer "F.Cu") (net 42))
 (segment (start 105.2 63.7525) (end 102.9525 66) (width 1) (layer "F.Cu") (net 42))
 (segment (start 105.2 63.7525) (end 105.2 31.8) (width 1) (layer "F.Cu") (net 42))
 (segment (start 96.015 66) (end 95.42 65.405) (width 1) (layer "F.Cu") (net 42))
 (segment (start 88.5 28.306802) (end 88.5 27) (width 1.5) (layer "F.Cu") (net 19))
 (segment (start 94.693198 34.5) (end 88.5 28.306802) (width 1.5) (layer "F.Cu") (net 19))
 (segment (start 96.5 34.5) (end 94.693198 34.5) (width 1.5) (layer "F.Cu") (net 19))
 (segment (start 92 27) (end 91 27) (width 1.5) (layer "F.Cu") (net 18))
 (segment (start 99.5 31.5) (end 96.5 31.5) (width 1.5) (layer "F.Cu") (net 18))
 (segment (start 96.5 31.5) (end 92 27) (width 1.5) (layer "F.Cu") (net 18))
 (segment (start 102.5 34.5) (end 99.5 31.5) (width 1.5) (layer "F.Cu") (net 18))
 (segment (start 73.643962 52) (end 72.253962 53.39) (width 1.5) (layer "F.Cu") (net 15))
 (segment (start 78 52) (end 73.643962 52) (width 1.5) (layer "F.Cu") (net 15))
 (segment (start 72.253962 53.39) (end 70.97 53.39) (width 1.5) (layer "F.Cu") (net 15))
 (segment (start 70.97 55.93) (end 72.384213 55.93) (width 1.5) (layer "F.Cu") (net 16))
 (segment (start 72.384213 55.93) (end 73.454213 57) (width 1.5) (layer "F.Cu") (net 16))
 (segment (start 73.454213 57) (end 78 57) (width 1.5) (layer "F.Cu") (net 16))
 (segment (start 73.081598 58.47) (end 77.051598 54.5) (width 1.5) (layer "B.Cu") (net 17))
 (segment (start 70.97 58.47) (end 73.081598 58.47) (width 1.5) (layer "B.Cu") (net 17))
 (segment (start 77.051598 54.5) (end 78 54.5) (width 1.5) (layer "B.Cu") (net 17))
 (segment (start 70.97 50.85) (end 75.701598 50.85) (width 1.5) (layer "B.Cu") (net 14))
 (segment (start 75.701598 50.85) (end 77.051598 49.5) (width 1.5) (layer "B.Cu") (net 14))
 (segment (start 77.051598 49.5) (end 78 49.5) (width 1.5) (layer "B.Cu") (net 14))
 (segment (start 84.88 43) (end 92.88 51) (width 0.5) (layer "B.Cu") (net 23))
 (segment (start 57.502692 43) (end 84.88 43) (width 0.5) (layer "B.Cu") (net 23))
 (segment (start 53.792692 39.29) (end 57.502692 43) (width 0.5) (layer "B.Cu") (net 23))
 (segment (start 50 39.29) (end 53.792692 39.29) (width 0.5) (layer "B.Cu") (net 23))
 (segment (start 77 36) (end 86 27) (width 0.5) (layer "B.Cu") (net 25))
 (segment (start 50 34.21) (end 51.13137 34.21) (width 0.5) (layer "B.Cu") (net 25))
 (segment (start 52.92137 36) (end 77 36) (width 0.5) (layer "B.Cu") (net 25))
 (segment (start 51.13137 34.21) (end 52.92137 36) (width 0.5) (layer "B.Cu") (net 25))
 (segment (start 88.7 58.28) (end 86.5 56.08) (width 1) (layer "F.Cu") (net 3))
 (segment (start 88.7 64.5) (end 88.7 58.28) (width 1) (layer "F.Cu") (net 3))
 (segment (start 81.57 61.01) (end 70.97 61.01) (width 1) (layer "B.Cu") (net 3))
 (segment (start 86.5 56.08) (end 81.57 61.01) (width 1) (layer "B.Cu") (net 3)))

